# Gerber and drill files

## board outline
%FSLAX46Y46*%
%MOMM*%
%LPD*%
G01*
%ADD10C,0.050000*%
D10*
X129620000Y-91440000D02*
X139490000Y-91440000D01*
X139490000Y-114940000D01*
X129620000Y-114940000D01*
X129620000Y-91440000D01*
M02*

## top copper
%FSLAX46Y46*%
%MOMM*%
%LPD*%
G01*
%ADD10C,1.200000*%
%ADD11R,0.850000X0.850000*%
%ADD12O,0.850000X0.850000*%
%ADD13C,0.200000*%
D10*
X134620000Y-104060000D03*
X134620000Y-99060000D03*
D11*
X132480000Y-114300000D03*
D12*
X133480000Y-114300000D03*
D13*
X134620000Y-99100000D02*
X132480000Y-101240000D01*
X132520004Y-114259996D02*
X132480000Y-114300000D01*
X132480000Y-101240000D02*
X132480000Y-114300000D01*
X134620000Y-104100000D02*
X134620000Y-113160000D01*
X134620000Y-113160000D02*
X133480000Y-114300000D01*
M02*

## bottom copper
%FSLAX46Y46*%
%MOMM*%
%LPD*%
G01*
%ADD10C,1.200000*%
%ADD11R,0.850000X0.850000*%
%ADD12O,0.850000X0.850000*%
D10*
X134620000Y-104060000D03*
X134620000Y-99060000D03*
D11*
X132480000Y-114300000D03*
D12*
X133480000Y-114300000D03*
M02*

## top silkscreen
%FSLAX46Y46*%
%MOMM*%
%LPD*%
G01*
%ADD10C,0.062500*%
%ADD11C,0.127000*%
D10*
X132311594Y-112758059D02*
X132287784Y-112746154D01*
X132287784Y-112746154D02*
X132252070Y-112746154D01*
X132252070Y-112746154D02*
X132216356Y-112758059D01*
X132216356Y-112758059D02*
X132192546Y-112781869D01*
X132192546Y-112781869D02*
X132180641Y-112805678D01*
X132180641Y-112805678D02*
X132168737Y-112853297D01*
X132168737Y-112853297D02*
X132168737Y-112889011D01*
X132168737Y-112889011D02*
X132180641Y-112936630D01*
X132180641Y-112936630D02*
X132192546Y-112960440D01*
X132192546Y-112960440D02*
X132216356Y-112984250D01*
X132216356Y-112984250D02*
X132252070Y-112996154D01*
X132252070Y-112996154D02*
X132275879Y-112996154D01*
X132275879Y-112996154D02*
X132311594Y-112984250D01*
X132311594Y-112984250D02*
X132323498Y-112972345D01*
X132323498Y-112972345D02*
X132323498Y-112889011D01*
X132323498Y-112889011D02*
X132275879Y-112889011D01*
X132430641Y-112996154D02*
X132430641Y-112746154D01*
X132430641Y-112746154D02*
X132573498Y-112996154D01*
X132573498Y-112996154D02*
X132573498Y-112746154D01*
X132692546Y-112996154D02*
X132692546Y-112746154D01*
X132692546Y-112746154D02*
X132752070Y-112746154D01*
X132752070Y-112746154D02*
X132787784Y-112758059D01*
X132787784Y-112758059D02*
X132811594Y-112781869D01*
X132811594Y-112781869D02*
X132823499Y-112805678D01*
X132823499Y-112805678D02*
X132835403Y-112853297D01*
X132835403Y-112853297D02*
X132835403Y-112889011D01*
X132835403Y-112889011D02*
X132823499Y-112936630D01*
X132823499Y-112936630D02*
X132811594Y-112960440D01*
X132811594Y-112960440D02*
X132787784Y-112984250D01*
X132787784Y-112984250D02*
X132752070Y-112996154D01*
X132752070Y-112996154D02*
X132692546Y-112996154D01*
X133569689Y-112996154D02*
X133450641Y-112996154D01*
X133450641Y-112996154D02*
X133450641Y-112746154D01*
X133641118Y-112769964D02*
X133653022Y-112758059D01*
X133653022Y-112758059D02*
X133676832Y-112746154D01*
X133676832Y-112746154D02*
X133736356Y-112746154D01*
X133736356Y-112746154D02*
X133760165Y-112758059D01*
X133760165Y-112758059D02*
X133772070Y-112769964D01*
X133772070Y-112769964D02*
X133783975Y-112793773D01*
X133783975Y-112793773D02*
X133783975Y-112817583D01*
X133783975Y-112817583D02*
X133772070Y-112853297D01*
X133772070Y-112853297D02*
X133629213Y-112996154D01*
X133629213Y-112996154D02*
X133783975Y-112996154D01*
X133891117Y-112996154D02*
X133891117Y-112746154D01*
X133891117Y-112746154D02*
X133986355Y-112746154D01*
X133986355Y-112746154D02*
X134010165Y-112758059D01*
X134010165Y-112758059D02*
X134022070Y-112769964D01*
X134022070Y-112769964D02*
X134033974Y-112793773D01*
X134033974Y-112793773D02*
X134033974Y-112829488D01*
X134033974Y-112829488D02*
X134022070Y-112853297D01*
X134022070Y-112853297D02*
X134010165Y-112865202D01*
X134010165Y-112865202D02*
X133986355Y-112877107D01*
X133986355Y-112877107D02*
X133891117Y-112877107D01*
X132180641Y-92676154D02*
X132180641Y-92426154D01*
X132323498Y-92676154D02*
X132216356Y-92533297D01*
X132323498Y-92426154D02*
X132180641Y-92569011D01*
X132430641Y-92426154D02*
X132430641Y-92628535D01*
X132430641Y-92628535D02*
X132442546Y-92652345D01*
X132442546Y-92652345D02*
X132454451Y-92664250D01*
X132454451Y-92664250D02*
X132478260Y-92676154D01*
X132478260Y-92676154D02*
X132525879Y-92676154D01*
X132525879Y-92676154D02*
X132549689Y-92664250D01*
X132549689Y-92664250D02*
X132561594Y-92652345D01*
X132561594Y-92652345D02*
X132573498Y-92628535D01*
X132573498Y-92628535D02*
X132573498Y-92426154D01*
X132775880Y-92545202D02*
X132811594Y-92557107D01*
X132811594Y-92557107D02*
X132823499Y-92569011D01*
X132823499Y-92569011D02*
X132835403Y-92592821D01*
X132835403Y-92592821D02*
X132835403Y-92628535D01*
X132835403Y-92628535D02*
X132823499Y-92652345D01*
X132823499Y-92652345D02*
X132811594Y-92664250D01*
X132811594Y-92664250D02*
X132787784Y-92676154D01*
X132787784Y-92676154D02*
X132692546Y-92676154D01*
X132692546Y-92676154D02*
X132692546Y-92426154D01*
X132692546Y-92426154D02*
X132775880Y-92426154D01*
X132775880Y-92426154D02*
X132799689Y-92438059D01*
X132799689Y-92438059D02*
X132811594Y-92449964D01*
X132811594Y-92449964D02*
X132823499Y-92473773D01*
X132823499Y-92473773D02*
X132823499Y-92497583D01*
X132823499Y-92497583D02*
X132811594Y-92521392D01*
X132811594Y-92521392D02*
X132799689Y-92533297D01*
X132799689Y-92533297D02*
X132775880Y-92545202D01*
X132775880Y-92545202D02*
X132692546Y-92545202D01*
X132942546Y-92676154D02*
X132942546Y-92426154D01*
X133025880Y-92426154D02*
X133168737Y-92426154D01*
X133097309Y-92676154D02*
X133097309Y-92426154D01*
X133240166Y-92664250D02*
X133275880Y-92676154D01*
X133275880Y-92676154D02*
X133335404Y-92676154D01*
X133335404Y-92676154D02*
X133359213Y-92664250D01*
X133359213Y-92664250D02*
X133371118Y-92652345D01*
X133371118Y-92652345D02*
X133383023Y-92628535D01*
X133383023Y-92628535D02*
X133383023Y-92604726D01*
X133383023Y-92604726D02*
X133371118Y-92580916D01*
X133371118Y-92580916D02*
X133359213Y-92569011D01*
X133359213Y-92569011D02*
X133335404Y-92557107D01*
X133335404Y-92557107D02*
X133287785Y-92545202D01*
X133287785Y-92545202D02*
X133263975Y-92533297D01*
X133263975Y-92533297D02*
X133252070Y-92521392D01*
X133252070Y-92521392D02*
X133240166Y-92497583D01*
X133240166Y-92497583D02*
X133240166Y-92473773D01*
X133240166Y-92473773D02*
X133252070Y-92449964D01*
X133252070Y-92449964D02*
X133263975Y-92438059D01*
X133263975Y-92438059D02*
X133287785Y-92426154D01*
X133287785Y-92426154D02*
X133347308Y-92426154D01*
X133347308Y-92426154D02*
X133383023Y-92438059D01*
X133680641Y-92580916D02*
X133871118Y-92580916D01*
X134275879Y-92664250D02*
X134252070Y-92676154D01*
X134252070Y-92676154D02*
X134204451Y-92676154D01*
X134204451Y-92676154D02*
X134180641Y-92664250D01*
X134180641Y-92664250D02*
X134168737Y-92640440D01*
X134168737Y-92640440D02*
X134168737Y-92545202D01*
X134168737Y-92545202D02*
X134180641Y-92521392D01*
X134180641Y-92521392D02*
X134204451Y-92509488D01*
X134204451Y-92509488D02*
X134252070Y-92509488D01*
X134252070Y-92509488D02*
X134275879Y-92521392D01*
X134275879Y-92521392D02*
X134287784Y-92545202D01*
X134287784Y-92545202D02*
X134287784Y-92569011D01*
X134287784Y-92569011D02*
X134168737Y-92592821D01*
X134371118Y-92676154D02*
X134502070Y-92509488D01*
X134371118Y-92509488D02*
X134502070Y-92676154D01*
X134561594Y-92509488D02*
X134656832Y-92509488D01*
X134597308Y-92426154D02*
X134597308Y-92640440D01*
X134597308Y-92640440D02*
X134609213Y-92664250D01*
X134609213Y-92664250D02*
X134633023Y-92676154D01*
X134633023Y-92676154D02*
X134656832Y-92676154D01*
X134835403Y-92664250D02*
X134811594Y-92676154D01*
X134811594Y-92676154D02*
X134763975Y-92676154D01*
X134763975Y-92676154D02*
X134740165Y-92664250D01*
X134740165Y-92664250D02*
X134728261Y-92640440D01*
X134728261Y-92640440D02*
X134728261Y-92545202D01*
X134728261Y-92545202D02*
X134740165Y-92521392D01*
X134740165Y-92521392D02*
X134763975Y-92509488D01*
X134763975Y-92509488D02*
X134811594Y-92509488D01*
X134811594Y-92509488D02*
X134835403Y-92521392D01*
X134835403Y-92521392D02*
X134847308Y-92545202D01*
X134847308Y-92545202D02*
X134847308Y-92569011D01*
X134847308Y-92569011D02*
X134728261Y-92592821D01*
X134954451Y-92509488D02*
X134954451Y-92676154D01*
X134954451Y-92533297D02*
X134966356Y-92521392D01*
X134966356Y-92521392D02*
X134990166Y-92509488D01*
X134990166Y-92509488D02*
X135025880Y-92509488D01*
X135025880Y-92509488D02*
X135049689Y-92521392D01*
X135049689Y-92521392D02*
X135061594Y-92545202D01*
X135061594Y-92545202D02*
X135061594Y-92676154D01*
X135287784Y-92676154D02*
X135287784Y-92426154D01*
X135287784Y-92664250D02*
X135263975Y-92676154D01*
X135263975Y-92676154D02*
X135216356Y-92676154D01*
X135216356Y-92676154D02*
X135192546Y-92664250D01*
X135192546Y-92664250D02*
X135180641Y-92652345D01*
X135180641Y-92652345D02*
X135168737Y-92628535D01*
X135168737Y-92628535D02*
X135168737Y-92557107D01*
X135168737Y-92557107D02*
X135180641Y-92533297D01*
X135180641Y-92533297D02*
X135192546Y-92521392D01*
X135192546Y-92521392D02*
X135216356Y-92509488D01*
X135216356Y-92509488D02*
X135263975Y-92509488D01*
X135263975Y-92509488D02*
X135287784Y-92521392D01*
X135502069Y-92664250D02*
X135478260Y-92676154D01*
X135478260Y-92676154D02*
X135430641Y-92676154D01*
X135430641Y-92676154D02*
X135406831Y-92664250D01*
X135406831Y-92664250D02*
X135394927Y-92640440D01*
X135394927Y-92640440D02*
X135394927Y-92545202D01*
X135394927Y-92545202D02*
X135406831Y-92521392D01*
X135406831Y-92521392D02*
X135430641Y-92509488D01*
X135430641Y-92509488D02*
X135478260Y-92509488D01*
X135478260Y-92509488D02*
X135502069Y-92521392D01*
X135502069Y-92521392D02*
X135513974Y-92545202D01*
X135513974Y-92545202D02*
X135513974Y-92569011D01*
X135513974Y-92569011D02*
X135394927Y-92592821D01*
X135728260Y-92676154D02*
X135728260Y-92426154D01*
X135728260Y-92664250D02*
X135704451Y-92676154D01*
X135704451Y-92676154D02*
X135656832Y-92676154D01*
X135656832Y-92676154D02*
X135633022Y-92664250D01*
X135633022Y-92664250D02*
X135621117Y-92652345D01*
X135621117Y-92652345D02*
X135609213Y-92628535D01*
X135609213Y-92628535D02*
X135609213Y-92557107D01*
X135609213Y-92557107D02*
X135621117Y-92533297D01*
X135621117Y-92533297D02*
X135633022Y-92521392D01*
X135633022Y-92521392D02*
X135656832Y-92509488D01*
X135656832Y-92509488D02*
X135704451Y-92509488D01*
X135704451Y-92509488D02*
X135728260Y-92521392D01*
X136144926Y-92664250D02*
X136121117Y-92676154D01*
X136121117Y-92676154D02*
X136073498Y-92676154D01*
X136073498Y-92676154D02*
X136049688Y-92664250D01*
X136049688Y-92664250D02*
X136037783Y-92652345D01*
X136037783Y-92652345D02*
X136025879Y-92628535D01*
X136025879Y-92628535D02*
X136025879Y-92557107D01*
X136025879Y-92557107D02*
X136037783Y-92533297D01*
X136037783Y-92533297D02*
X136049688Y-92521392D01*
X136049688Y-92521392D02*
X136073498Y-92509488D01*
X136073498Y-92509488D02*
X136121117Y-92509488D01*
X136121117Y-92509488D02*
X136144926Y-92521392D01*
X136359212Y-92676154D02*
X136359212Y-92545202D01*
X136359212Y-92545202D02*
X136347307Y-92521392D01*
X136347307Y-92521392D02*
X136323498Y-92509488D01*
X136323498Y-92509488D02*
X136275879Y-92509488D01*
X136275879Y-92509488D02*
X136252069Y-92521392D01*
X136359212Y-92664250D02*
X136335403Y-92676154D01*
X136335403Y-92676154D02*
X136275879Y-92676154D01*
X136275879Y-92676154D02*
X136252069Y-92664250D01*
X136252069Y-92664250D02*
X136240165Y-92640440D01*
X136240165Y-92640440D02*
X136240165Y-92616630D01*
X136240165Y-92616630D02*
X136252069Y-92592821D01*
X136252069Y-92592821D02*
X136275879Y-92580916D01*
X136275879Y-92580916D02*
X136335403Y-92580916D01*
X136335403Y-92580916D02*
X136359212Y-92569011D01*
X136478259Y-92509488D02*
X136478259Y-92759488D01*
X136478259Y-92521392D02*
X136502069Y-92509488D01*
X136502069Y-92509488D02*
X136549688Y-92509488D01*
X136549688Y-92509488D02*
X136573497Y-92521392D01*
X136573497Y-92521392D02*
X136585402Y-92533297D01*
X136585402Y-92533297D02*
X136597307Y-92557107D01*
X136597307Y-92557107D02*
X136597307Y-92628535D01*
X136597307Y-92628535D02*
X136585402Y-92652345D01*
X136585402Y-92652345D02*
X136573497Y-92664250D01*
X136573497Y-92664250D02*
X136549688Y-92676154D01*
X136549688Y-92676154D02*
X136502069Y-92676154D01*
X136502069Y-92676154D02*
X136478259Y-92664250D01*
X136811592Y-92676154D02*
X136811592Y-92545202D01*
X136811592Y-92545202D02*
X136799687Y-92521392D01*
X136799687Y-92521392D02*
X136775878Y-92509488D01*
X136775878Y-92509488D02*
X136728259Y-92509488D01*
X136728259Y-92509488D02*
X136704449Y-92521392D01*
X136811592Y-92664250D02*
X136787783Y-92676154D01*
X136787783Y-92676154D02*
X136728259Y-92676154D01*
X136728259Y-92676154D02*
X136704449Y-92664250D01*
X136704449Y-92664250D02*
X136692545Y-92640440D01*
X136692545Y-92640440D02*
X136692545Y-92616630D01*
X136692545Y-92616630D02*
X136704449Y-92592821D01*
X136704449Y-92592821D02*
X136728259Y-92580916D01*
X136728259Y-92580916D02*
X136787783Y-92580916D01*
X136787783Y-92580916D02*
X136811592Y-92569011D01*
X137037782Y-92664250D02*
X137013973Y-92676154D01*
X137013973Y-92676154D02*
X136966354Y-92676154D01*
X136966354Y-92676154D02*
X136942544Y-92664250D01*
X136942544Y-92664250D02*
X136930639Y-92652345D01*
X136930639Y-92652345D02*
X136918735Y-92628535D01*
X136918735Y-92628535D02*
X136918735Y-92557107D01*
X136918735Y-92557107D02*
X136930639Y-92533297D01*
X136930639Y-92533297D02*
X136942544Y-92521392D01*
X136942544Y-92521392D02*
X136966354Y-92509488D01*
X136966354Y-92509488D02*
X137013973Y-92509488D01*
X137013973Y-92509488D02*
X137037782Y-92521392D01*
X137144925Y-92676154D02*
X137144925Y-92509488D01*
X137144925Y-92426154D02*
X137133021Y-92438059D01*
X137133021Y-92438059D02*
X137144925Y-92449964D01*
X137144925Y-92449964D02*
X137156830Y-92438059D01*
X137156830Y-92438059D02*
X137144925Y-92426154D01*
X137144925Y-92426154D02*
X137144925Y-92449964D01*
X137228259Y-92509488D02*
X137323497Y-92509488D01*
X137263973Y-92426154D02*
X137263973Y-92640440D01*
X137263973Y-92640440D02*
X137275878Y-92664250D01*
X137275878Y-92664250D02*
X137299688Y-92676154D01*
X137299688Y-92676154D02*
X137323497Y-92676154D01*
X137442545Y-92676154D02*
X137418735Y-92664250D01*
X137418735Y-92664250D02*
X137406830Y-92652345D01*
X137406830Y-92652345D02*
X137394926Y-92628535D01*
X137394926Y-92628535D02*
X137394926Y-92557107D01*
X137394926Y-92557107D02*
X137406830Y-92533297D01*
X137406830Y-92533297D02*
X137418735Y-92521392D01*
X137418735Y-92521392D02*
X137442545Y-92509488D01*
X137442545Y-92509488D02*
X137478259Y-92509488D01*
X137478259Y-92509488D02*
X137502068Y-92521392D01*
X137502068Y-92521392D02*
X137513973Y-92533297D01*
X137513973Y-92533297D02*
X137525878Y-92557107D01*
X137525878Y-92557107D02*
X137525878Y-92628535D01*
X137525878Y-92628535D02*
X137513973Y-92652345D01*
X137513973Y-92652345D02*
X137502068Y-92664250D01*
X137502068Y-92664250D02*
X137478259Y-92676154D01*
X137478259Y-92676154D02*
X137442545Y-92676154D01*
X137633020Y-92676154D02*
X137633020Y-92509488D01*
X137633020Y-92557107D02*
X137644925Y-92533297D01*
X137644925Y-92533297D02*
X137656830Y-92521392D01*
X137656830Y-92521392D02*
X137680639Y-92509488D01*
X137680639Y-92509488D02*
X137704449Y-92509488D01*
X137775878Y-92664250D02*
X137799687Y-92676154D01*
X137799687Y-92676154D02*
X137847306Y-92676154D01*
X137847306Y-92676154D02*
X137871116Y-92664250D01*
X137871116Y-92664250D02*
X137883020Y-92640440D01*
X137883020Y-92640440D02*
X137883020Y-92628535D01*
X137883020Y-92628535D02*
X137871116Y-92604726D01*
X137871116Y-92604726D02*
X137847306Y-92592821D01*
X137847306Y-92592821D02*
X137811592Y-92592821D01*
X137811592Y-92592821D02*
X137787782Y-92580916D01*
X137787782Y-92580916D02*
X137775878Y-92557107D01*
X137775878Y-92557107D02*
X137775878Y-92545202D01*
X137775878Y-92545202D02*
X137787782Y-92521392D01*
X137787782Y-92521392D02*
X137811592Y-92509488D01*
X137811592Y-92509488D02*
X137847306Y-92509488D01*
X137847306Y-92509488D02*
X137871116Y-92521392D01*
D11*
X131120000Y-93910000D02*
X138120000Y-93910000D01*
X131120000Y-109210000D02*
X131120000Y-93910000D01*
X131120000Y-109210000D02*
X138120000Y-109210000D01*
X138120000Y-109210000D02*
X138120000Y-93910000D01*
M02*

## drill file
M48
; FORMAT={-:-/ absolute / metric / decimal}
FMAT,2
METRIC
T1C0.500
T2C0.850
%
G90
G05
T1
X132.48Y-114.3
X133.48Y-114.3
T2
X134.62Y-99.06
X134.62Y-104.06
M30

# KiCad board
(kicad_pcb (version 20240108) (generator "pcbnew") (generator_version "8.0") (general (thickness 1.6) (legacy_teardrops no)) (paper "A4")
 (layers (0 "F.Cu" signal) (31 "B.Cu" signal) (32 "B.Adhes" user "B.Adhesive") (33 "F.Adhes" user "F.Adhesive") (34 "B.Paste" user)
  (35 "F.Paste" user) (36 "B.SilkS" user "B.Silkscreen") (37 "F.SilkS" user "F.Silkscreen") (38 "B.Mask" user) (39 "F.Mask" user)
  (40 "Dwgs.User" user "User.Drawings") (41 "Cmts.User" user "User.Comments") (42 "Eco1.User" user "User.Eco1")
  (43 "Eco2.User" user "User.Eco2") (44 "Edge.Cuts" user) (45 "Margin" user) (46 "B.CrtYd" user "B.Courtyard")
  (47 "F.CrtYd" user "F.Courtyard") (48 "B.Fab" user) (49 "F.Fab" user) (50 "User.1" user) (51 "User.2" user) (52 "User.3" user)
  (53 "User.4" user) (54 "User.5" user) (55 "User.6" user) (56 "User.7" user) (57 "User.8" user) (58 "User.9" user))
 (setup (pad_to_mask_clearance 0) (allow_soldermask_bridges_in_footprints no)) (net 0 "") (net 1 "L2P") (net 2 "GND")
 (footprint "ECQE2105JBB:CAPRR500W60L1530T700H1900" (layer "F.Cu") (at 134.62 101.56 90)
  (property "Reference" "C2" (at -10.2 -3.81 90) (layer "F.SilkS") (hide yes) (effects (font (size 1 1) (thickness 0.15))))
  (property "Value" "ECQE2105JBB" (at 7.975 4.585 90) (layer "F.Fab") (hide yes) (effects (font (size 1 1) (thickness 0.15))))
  (fp_line (start 7.65 -3.5) (end 7.65 3.5) (stroke (width 0.127) (type solid)) (layer "F.SilkS"))
  (fp_line (start -7.65 -3.5) (end 7.65 -3.5) (stroke (width 0.127) (type solid)) (layer "F.SilkS"))
  (fp_line (start -7.65 -3.5) (end -7.65 3.5) (stroke (width 0.127) (type solid)) (layer "F.SilkS"))
  (fp_line (start -7.65 3.5) (end 7.65 3.5) (stroke (width 0.127) (type solid)) (layer "F.SilkS"))
  (pad "1" thru_hole circle (at -2.5 0 90) (size 1.2 1.2) (drill 0.85) (layers "*.Cu" "*.Mask") (remove_unused_layers no) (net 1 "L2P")
   (solder_mask_margin 0.102))
  (pad "2" thru_hole circle (at 2.5 0 90) (size 1.2 1.2) (drill 0.85) (layers "*.Cu" "*.Mask") (remove_unused_layers no) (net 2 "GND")
   (solder_mask_margin 0.102)))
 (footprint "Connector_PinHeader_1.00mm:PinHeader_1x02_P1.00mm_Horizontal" (layer "B.Cu") (at 132.48 114.3 -90)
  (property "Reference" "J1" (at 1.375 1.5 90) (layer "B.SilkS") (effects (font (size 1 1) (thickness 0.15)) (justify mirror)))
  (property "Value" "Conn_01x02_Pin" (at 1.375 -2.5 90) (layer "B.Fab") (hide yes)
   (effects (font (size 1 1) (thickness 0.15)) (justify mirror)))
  (pad "1" thru_hole rect (at 0 0 270) (size 0.85 0.85) (drill 0.5) (layers "*.Cu" "*.Mask") (remove_unused_layers no) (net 2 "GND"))
  (pad "2" thru_hole oval (at 0 -1 270) (size 0.85 0.85) (drill 0.5) (layers "*.Cu" "*.Mask") (remove_unused_layers no) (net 1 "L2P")))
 (gr_rect (start 129.62 91.44) (end 139.49 114.94) (stroke (width 0.05) (type default)) (fill none) (layer "Edge.Cuts"))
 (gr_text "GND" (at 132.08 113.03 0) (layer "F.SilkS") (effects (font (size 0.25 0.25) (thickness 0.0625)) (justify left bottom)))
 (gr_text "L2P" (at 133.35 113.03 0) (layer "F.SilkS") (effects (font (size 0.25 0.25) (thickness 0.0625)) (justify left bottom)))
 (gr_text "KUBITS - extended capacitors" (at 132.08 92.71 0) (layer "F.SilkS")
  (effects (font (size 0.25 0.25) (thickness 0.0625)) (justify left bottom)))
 (segment (start 134.62 99.1) (end 132.48 101.24) (width 0.2) (layer "F.Cu") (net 2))
 (segment (start 132.520004 114.259996) (end 132.48 114.3) (width 0.2) (layer "F.Cu") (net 2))
 (segment (start 132.48 101.24) (end 132.48 114.3) (width 0.2) (layer "F.Cu") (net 2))
 (segment (start 134.62 104.1) (end 134.62 113.16) (width 0.2) (layer "F.Cu") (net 1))
 (segment (start 134.62 113.16) (end 133.48 114.3) (width 0.2) (layer "F.Cu") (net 1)))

